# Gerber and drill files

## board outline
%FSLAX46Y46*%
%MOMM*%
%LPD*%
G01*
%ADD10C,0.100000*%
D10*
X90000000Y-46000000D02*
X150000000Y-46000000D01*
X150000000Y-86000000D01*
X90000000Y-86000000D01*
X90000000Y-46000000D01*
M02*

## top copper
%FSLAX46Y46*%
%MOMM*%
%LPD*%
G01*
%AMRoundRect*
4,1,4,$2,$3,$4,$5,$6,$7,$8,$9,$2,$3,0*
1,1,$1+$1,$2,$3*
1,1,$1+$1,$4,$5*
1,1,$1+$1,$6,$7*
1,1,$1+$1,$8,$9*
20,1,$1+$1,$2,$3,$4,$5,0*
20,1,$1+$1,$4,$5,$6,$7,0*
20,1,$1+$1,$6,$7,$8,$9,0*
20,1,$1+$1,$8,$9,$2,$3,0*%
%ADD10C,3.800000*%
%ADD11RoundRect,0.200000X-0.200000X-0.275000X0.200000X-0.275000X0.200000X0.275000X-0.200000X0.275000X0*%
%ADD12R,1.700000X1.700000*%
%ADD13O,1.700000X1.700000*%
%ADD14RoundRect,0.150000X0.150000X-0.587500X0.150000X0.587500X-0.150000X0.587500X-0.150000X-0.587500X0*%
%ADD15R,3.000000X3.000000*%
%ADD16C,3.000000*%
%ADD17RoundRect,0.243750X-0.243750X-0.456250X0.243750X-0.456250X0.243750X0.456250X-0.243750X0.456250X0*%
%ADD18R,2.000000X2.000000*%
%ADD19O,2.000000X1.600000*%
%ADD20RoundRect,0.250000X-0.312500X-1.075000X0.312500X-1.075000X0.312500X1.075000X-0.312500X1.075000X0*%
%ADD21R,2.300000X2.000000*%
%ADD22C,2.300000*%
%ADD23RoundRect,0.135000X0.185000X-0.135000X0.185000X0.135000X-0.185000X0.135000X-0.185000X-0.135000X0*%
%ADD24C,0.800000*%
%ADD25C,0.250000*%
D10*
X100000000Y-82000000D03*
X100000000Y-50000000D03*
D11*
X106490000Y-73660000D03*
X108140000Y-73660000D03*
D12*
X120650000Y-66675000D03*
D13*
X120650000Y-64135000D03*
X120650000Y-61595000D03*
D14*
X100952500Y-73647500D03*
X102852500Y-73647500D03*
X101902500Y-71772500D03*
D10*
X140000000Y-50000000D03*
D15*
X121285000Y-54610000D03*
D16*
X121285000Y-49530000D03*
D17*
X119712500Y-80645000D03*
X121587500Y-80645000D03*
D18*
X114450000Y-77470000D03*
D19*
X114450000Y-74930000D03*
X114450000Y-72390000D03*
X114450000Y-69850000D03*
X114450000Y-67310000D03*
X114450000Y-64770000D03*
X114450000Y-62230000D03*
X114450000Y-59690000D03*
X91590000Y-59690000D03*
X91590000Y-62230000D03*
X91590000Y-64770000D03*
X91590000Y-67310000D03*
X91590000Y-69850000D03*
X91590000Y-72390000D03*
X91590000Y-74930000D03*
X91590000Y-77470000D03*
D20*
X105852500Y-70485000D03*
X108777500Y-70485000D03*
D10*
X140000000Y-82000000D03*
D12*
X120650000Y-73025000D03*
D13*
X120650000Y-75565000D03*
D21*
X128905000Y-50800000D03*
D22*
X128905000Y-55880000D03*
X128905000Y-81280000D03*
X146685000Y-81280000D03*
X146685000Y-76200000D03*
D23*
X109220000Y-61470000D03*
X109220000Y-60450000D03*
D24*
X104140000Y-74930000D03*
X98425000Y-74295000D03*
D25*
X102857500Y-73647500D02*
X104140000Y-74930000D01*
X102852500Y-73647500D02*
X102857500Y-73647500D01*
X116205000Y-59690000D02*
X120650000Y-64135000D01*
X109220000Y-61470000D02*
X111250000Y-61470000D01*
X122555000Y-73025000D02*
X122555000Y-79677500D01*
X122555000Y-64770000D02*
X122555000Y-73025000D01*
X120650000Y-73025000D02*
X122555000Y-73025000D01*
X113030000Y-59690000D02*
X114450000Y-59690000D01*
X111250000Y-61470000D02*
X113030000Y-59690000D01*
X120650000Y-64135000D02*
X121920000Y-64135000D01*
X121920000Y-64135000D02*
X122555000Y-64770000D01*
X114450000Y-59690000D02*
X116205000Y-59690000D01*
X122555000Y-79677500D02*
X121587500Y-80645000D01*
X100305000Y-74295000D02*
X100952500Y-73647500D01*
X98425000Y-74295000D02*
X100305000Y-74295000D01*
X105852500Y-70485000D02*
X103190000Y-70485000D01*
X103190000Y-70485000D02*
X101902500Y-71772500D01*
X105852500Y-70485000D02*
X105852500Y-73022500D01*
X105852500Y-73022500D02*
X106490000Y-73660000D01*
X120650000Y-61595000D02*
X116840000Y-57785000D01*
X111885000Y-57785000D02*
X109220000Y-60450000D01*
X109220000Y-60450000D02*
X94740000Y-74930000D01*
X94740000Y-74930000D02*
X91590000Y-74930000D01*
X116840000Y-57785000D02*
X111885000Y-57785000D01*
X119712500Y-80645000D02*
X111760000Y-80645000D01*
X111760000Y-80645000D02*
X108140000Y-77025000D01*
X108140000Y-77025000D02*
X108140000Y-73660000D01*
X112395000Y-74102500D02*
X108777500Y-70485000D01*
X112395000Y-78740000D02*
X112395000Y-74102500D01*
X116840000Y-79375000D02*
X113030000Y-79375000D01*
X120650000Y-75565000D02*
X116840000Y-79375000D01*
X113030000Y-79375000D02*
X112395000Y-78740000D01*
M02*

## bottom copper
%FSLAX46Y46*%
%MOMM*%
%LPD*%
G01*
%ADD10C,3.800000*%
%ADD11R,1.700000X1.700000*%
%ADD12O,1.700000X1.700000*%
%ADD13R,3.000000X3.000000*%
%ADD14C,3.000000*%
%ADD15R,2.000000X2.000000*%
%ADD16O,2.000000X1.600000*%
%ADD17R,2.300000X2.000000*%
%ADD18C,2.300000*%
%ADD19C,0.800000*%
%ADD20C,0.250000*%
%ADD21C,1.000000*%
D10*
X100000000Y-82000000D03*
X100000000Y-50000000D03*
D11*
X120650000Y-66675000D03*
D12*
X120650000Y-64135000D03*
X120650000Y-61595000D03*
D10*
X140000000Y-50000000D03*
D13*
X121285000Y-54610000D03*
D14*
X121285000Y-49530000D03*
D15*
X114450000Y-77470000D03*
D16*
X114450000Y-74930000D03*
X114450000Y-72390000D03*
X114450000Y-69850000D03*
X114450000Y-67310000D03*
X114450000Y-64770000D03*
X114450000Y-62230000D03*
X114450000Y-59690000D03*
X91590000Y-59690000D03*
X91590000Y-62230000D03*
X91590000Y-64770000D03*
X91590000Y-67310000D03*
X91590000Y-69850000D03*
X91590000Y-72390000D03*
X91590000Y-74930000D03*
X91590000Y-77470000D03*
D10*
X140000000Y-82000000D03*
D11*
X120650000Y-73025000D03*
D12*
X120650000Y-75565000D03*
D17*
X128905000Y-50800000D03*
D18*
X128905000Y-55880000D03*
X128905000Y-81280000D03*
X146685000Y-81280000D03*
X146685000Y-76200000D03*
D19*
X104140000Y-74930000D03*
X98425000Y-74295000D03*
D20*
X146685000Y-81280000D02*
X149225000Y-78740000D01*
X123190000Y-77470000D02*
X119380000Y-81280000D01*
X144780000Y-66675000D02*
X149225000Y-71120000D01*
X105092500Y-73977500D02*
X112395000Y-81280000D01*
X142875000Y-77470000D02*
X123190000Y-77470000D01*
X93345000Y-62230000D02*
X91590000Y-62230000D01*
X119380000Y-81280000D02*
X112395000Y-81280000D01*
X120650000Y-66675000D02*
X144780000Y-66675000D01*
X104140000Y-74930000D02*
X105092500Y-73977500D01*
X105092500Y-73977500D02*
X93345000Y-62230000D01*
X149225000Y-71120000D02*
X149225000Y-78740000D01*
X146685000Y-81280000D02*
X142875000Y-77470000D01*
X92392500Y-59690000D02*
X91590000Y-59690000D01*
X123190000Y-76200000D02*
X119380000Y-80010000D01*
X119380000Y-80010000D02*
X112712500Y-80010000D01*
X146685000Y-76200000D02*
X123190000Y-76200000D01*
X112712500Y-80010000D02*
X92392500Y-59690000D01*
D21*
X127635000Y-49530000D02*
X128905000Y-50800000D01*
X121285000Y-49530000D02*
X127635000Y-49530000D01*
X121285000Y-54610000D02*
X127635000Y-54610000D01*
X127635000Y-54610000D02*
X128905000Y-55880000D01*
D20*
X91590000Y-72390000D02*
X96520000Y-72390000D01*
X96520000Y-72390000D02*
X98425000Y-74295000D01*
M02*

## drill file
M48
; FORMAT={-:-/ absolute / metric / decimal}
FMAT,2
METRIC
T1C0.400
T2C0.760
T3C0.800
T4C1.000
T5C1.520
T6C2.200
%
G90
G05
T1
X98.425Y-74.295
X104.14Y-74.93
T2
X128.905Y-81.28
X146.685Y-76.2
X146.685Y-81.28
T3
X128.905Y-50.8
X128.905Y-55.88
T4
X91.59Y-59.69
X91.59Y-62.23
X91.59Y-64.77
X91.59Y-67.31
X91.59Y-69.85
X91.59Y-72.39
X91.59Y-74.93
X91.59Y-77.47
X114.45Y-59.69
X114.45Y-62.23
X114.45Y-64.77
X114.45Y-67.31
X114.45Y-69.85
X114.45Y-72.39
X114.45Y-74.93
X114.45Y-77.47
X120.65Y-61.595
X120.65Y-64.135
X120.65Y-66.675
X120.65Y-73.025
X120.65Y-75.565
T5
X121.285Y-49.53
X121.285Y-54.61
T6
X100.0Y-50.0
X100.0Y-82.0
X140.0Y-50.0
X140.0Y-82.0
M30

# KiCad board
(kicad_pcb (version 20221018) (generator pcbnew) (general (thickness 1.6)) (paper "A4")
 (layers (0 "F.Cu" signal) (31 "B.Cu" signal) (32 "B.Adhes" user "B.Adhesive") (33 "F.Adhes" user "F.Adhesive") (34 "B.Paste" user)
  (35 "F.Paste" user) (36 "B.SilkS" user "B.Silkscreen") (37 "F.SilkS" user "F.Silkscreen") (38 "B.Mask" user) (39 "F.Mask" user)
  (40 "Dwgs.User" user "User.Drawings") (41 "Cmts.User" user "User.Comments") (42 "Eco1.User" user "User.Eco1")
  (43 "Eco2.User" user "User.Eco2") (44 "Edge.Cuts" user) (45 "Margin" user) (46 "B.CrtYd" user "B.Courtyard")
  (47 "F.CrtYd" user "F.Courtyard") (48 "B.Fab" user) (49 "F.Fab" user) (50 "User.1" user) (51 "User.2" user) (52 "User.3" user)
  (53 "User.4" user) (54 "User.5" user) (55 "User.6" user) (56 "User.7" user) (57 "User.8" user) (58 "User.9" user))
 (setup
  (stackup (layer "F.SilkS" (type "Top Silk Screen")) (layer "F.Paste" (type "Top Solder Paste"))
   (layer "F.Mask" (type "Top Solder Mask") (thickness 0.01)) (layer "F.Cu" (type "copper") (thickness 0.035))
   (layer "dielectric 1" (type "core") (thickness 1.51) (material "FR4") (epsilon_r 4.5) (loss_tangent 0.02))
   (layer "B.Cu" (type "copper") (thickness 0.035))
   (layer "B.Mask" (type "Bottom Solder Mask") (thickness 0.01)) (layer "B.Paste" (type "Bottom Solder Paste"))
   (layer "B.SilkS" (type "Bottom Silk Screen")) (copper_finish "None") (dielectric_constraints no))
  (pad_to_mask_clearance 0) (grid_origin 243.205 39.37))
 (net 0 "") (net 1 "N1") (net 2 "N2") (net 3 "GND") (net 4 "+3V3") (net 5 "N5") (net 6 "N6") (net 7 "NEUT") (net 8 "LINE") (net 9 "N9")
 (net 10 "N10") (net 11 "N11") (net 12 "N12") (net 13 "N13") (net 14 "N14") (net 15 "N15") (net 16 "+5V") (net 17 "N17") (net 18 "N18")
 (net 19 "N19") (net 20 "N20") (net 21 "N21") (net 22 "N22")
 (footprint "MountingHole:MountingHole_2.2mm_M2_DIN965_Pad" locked (layer "F.Cu") (at 100 82)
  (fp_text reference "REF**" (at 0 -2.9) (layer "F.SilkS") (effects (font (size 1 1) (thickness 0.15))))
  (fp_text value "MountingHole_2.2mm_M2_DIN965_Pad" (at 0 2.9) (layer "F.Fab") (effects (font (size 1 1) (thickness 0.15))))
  (pad "1" thru_hole circle locked (at 0 0) (size 3.8 3.8) (drill 2.2) (layers "*.Cu" "*.Mask")))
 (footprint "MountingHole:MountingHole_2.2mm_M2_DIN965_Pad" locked (layer "F.Cu") (at 100 50)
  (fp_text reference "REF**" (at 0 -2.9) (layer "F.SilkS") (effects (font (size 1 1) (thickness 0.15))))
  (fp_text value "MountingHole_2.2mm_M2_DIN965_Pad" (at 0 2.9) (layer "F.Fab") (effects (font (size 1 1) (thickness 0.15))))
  (pad "1" thru_hole circle locked (at 0 0) (size 3.8 3.8) (drill 2.2) (layers "*.Cu" "*.Mask")))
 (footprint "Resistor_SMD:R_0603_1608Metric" (layer "F.Cu") (at 107.315 73.66)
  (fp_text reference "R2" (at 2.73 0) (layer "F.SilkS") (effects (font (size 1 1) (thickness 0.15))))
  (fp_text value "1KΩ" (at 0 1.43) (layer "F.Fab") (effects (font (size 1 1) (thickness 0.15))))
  (pad "1" smd roundrect (at -0.825 0) (size 0.8 0.95) (layers "F.Cu" "F.Paste" "F.Mask") (roundrect_rratio 0.25) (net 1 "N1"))
  (pad "2" smd roundrect (at 0.825 0) (size 0.8 0.95) (layers "F.Cu" "F.Paste" "F.Mask") (roundrect_rratio 0.25) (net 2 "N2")))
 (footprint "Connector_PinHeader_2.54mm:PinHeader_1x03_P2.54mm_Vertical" (layer "F.Cu") (at 120.65 66.675 180)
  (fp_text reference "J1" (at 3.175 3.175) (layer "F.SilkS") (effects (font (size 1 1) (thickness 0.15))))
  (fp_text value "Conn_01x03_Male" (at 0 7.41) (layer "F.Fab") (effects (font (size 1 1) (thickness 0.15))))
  (pad "1" thru_hole rect (at 0 0 180) (size 1.7 1.7) (drill 1) (layers "*.Cu" "*.Mask") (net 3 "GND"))
  (pad "2" thru_hole oval (at 0 2.54 180) (size 1.7 1.7) (drill 1) (layers "*.Cu" "*.Mask") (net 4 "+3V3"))
  (pad "3" thru_hole oval (at 0 5.08 180) (size 1.7 1.7) (drill 1) (layers "*.Cu" "*.Mask") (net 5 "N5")))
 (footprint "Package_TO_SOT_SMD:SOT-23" (layer "F.Cu") (at 101.9025 72.71 90)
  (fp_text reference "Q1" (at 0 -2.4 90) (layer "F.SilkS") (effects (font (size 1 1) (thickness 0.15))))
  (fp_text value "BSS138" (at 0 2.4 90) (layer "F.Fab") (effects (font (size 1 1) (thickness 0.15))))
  (pad "1" smd roundrect (at -0.9375 -0.95 90) (size 1.475 0.6) (layers "F.Cu" "F.Paste" "F.Mask") (roundrect_rratio 0.25) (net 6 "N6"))
  (pad "2" smd roundrect (at -0.9375 0.95 90) (size 1.475 0.6) (layers "F.Cu" "F.Paste" "F.Mask") (roundrect_rratio 0.25) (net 3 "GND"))
  (pad "3" smd roundrect (at 0.9375 0 90) (size 1.475 0.6) (layers "F.Cu" "F.Paste" "F.Mask") (roundrect_rratio 0.25) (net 1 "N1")))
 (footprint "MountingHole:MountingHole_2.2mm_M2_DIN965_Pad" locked (layer "F.Cu") (at 140 50)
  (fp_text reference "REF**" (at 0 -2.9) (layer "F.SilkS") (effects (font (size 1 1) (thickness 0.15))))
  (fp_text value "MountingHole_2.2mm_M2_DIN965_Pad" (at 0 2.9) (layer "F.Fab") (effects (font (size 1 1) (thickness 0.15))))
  (pad "1" thru_hole circle locked (at 0 0) (size 3.8 3.8) (drill 2.2) (layers "*.Cu" "*.Mask")))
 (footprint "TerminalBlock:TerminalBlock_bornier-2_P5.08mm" (layer "F.Cu") (at 121.285 54.61 90)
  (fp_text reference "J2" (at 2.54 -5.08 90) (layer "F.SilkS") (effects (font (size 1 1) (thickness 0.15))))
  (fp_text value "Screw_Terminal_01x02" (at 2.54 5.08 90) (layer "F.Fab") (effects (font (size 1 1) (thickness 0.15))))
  (pad "1" thru_hole rect (at 0 0 90) (size 3 3) (drill 1.52) (layers "*.Cu" "*.Mask") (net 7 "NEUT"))
  (pad "2" thru_hole circle (at 5.08 0 90) (size 3 3) (drill 1.52) (layers "*.Cu" "*.Mask") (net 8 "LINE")))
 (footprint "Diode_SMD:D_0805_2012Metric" (layer "F.Cu") (at 120.65 80.645)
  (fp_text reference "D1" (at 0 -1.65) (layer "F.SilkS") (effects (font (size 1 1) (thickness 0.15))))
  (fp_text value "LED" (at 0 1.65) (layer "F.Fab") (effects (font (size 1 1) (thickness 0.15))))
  (pad "1" smd roundrect (at -0.9375 0) (size 0.975 1.4) (layers "F.Cu" "F.Paste" "F.Mask") (roundrect_rratio 0.25) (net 2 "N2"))
  (pad "2" smd roundrect (at 0.9375 0) (size 0.975 1.4) (layers "F.Cu" "F.Paste" "F.Mask") (roundrect_rratio 0.25) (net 4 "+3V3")))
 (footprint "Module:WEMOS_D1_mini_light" (layer "F.Cu") (at 114.45 77.47 180)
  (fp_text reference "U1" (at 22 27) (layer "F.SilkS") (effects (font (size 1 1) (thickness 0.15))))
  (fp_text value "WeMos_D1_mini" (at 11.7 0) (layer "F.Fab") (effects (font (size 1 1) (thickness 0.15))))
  (pad "1" thru_hole rect (at 0 0 180) (size 2 2) (drill 1) (layers "*.Cu" "*.Mask") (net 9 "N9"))
  (pad "2" thru_hole oval (at 0 2.54 180) (size 2 1.6) (drill 1) (layers "*.Cu" "*.Mask") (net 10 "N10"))
  (pad "3" thru_hole oval (at 0 5.08 180) (size 2 1.6) (drill 1) (layers "*.Cu" "*.Mask") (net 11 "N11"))
  (pad "4" thru_hole oval (at 0 7.62 180) (size 2 1.6) (drill 1) (layers "*.Cu" "*.Mask") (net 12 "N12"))
  (pad "5" thru_hole oval (at 0 10.16 180) (size 2 1.6) (drill 1) (layers "*.Cu" "*.Mask") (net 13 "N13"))
  (pad "6" thru_hole oval (at 0 12.7 180) (size 2 1.6) (drill 1) (layers "*.Cu" "*.Mask") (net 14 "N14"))
  (pad "7" thru_hole oval (at 0 15.24 180) (size 2 1.6) (drill 1) (layers "*.Cu" "*.Mask") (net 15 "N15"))
  (pad "8" thru_hole oval (at 0 17.78 180) (size 2 1.6) (drill 1) (layers "*.Cu" "*.Mask") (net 4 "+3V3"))
  (pad "9" thru_hole oval (at 22.86 17.78 180) (size 2 1.6) (drill 1) (layers "*.Cu" "*.Mask") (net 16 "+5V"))
  (pad "10" thru_hole oval (at 22.86 15.24 180) (size 2 1.6) (drill 1) (layers "*.Cu" "*.Mask") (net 3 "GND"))
  (pad "11" thru_hole oval (at 22.86 12.7 180) (size 2 1.6) (drill 1) (layers "*.Cu" "*.Mask") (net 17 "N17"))
  (pad "12" thru_hole oval (at 22.86 10.16 180) (size 2 1.6) (drill 1) (layers "*.Cu" "*.Mask") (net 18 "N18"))
  (pad "13" thru_hole oval (at 22.86 7.62 180) (size 2 1.6) (drill 1) (layers "*.Cu" "*.Mask") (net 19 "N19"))
  (pad "14" thru_hole oval (at 22.86 5.08 180) (size 2 1.6) (drill 1) (layers "*.Cu" "*.Mask") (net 6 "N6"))
  (pad "15" thru_hole oval (at 22.86 2.54 180) (size 2 1.6) (drill 1) (layers "*.Cu" "*.Mask") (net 5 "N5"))
  (pad "16" thru_hole oval (at 22.86 0 180) (size 2 1.6) (drill 1) (layers "*.Cu" "*.Mask") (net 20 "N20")))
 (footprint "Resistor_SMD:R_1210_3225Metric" (layer "F.Cu") (at 107.315 70.485)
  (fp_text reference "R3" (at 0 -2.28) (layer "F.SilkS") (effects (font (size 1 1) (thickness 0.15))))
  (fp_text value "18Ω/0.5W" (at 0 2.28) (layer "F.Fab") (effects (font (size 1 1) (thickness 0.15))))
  (pad "1" smd roundrect (at -1.4625 0) (size 1.125 2.65) (layers "F.Cu" "F.Paste" "F.Mask") (roundrect_rratio 0.2222222222) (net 1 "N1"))
  (pad "2" smd roundrect (at 1.4625 0) (size 1.125 2.65) (layers "F.Cu" "F.Paste" "F.Mask") (roundrect_rratio 0.2222222222) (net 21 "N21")))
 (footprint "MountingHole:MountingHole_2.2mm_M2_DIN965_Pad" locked (layer "F.Cu") (at 140 82)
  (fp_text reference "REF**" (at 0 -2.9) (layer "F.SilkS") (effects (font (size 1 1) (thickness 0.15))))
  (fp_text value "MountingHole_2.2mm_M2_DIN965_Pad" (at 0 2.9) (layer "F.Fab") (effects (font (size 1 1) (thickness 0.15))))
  (pad "1" thru_hole circle locked (at 0 0) (size 3.8 3.8) (drill 2.2) (layers "*.Cu" "*.Mask")))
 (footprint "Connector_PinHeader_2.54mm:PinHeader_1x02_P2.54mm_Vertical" (layer "F.Cu") (at 120.65 73.025)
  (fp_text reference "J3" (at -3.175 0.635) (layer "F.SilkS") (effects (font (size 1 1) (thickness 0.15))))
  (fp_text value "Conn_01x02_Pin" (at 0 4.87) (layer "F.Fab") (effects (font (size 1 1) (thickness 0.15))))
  (pad "1" thru_hole rect (at 0 0) (size 1.7 1.7) (drill 1) (layers "*.Cu" "*.Mask") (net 4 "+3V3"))
  (pad "2" thru_hole oval (at 0 2.54) (size 1.7 1.7) (drill 1) (layers "*.Cu" "*.Mask") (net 21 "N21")))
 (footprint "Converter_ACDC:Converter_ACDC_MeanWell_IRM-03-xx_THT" (layer "F.Cu") (at 128.905 50.8)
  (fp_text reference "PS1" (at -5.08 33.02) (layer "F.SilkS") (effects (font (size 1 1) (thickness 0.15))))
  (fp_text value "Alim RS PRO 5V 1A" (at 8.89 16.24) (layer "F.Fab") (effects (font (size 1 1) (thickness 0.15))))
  (pad "1" thru_hole rect (at 0 0) (size 2.3 2) (drill 0.8) (layers "*.Cu" "*.Mask") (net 8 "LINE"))
  (pad "3" thru_hole circle (at 0 5.08) (size 2.3 2.3) (drill 0.8) (layers "*.Cu" "*.Mask") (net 7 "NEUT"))
  (pad "5" thru_hole circle (at 0 30.48) (size 2.3 2.3) (drill 0.76) (layers "*.Cu" "*.Mask") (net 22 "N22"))
  (pad "14" thru_hole circle (at 17.78 30.48) (size 2.3 2.3) (drill 0.76) (layers "*.Cu" "*.Mask") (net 3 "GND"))
  (pad "16" thru_hole circle (at 17.78 25.4) (size 2.3 2.3) (drill 0.76) (layers "*.Cu" "*.Mask") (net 16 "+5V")))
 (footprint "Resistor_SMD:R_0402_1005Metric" (layer "F.Cu") (at 109.22 60.96 90)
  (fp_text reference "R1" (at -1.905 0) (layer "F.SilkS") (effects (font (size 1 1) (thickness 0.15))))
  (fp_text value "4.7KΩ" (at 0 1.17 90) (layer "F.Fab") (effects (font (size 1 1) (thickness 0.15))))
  (pad "1" smd roundrect (at -0.51 0 90) (size 0.54 0.64) (layers "F.Cu" "F.Paste" "F.Mask") (roundrect_rratio 0.25) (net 4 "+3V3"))
  (pad "2" smd roundrect (at 0.51 0 90) (size 0.54 0.64) (layers "F.Cu" "F.Paste" "F.Mask") (roundrect_rratio 0.25) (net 5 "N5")))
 (gr_rect locked (start 90 46) (end 150 86) (stroke (width 0.1) (type default)) (fill none) (layer "Edge.Cuts"))
 (segment (start 102.8575 73.6475) (end 104.14 74.93) (width 0.25) (layer "F.Cu") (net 3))
 (segment (start 102.8525 73.6475) (end 102.8575 73.6475) (width 0.25) (layer "F.Cu") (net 3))
 (via (at 104.14 74.93) (size 0.8) (drill 0.4) (layers "F.Cu" "B.Cu") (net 3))
 (segment (start 146.685 81.28) (end 149.225 78.74) (width 0.25) (layer "B.Cu") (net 3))
 (segment (start 123.19 77.47) (end 119.38 81.28) (width 0.25) (layer "B.Cu") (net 3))
 (segment (start 144.78 66.675) (end 149.225 71.12) (width 0.25) (layer "B.Cu") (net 3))
 (segment (start 105.0925 73.9775) (end 112.395 81.28) (width 0.25) (layer "B.Cu") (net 3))
 (segment (start 142.875 77.47) (end 123.19 77.47) (width 0.25) (layer "B.Cu") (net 3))
 (segment (start 93.345 62.23) (end 91.59 62.23) (width 0.25) (layer "B.Cu") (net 3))
 (segment (start 119.38 81.28) (end 112.395 81.28) (width 0.25) (layer "B.Cu") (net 3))
 (segment (start 120.65 66.675) (end 144.78 66.675) (width 0.25) (layer "B.Cu") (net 3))
 (segment (start 104.14 74.93) (end 105.0925 73.9775) (width 0.25) (layer "B.Cu") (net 3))
 (segment (start 105.0925 73.9775) (end 93.345 62.23) (width 0.25) (layer "B.Cu") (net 3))
 (segment (start 149.225 71.12) (end 149.225 78.74) (width 0.25) (layer "B.Cu") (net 3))
 (segment (start 146.685 81.28) (end 142.875 77.47) (width 0.25) (layer "B.Cu") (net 3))
 (segment (start 92.3925 59.69) (end 91.59 59.69) (width 0.25) (layer "B.Cu") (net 16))
 (segment (start 123.19 76.2) (end 119.38 80.01) (width 0.25) (layer "B.Cu") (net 16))
 (segment (start 119.38 80.01) (end 112.7125 80.01) (width 0.25) (layer "B.Cu") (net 16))
 (segment (start 146.685 76.2) (end 123.19 76.2) (width 0.25) (layer "B.Cu") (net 16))
 (segment (start 112.7125 80.01) (end 92.3925 59.69) (width 0.25) (layer "B.Cu") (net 16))
 (segment (start 116.205 59.69) (end 120.65 64.135) (width 0.25) (layer "F.Cu") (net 4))
 (segment (start 109.22 61.47) (end 111.25 61.47) (width 0.25) (layer "F.Cu") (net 4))
 (segment (start 122.555 73.025) (end 122.555 79.6775) (width 0.25) (layer "F.Cu") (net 4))
 (segment (start 122.555 64.77) (end 122.555 73.025) (width 0.25) (layer "F.Cu") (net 4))
 (segment (start 120.65 73.025) (end 122.555 73.025) (width 0.25) (layer "F.Cu") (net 4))
 (segment (start 113.03 59.69) (end 114.45 59.69) (width 0.25) (layer "F.Cu") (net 4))
 (segment (start 111.25 61.47) (end 113.03 59.69) (width 0.25) (layer "F.Cu") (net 4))
 (segment (start 120.65 64.135) (end 121.92 64.135) (width 0.25) (layer "F.Cu") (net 4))
 (segment (start 121.92 64.135) (end 122.555 64.77) (width 0.25) (layer "F.Cu") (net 4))
 (segment (start 114.45 59.69) (end 116.205 59.69) (width 0.25) (layer "F.Cu") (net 4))
 (segment (start 122.555 79.6775) (end 121.5875 80.645) (width 0.25) (layer "F.Cu") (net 4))
 (segment (start 127.635 49.53) (end 128.905 50.8) (width 1) (layer "B.Cu") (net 8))
 (segment (start 121.285 49.53) (end 127.635 49.53) (width 1) (layer "B.Cu") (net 8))
 (segment (start 121.285 54.61) (end 127.635 54.61) (width 1) (layer "B.Cu") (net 7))
 (segment (start 127.635 54.61) (end 128.905 55.88) (width 1) (layer "B.Cu") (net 7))
 (segment (start 100.305 74.295) (end 100.9525 73.6475) (width 0.25) (layer "F.Cu") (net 6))
 (segment (start 98.425 74.295) (end 100.305 74.295) (width 0.25) (layer "F.Cu") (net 6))
 (via (at 98.425 74.295) (size 0.8) (drill 0.4) (layers "F.Cu" "B.Cu") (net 6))
 (segment (start 91.59 72.39) (end 96.52 72.39) (width 0.25) (layer "B.Cu") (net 6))
 (segment (start 96.52 72.39) (end 98.425 74.295) (width 0.25) (layer "B.Cu") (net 6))
 (segment (start 105.8525 70.485) (end 103.19 70.485) (width 0.25) (layer "F.Cu") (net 1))
 (segment (start 103.19 70.485) (end 101.9025 71.7725) (width 0.25) (layer "F.Cu") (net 1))
 (segment (start 105.8525 70.485) (end 105.8525 73.0225) (width 0.25) (layer "F.Cu") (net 1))
 (segment (start 105.8525 73.0225) (end 106.49 73.66) (width 0.25) (layer "F.Cu") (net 1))
 (segment (start 120.65 61.595) (end 116.84 57.785) (width 0.25) (layer "F.Cu") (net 5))
 (segment (start 111.885 57.785) (end 109.22 60.45) (width 0.25) (layer "F.Cu") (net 5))
 (segment (start 109.22 60.45) (end 94.74 74.93) (width 0.25) (layer "F.Cu") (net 5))
 (segment (start 94.74 74.93) (end 91.59 74.93) (width 0.25) (layer "F.Cu") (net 5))
 (segment (start 116.84 57.785) (end 111.885 57.785) (width 0.25) (layer "F.Cu") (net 5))
 (segment (start 119.7125 80.645) (end 111.76 80.645) (width 0.25) (layer "F.Cu") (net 2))
 (segment (start 111.76 80.645) (end 108.14 77.025) (width 0.25) (layer "F.Cu") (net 2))
 (segment (start 108.14 77.025) (end 108.14 73.66) (width 0.25) (layer "F.Cu") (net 2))
 (segment (start 112.395 74.1025) (end 108.7775 70.485) (width 0.25) (layer "F.Cu") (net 21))
 (segment (start 112.395 78.74) (end 112.395 74.1025) (width 0.25) (layer "F.Cu") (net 21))
 (segment (start 116.84 79.375) (end 113.03 79.375) (width 0.25) (layer "F.Cu") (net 21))
 (segment (start 120.65 75.565) (end 116.84 79.375) (width 0.25) (layer "F.Cu") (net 21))
 (segment (start 113.03 79.375) (end 112.395 78.74) (width 0.25) (layer "F.Cu") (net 21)))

